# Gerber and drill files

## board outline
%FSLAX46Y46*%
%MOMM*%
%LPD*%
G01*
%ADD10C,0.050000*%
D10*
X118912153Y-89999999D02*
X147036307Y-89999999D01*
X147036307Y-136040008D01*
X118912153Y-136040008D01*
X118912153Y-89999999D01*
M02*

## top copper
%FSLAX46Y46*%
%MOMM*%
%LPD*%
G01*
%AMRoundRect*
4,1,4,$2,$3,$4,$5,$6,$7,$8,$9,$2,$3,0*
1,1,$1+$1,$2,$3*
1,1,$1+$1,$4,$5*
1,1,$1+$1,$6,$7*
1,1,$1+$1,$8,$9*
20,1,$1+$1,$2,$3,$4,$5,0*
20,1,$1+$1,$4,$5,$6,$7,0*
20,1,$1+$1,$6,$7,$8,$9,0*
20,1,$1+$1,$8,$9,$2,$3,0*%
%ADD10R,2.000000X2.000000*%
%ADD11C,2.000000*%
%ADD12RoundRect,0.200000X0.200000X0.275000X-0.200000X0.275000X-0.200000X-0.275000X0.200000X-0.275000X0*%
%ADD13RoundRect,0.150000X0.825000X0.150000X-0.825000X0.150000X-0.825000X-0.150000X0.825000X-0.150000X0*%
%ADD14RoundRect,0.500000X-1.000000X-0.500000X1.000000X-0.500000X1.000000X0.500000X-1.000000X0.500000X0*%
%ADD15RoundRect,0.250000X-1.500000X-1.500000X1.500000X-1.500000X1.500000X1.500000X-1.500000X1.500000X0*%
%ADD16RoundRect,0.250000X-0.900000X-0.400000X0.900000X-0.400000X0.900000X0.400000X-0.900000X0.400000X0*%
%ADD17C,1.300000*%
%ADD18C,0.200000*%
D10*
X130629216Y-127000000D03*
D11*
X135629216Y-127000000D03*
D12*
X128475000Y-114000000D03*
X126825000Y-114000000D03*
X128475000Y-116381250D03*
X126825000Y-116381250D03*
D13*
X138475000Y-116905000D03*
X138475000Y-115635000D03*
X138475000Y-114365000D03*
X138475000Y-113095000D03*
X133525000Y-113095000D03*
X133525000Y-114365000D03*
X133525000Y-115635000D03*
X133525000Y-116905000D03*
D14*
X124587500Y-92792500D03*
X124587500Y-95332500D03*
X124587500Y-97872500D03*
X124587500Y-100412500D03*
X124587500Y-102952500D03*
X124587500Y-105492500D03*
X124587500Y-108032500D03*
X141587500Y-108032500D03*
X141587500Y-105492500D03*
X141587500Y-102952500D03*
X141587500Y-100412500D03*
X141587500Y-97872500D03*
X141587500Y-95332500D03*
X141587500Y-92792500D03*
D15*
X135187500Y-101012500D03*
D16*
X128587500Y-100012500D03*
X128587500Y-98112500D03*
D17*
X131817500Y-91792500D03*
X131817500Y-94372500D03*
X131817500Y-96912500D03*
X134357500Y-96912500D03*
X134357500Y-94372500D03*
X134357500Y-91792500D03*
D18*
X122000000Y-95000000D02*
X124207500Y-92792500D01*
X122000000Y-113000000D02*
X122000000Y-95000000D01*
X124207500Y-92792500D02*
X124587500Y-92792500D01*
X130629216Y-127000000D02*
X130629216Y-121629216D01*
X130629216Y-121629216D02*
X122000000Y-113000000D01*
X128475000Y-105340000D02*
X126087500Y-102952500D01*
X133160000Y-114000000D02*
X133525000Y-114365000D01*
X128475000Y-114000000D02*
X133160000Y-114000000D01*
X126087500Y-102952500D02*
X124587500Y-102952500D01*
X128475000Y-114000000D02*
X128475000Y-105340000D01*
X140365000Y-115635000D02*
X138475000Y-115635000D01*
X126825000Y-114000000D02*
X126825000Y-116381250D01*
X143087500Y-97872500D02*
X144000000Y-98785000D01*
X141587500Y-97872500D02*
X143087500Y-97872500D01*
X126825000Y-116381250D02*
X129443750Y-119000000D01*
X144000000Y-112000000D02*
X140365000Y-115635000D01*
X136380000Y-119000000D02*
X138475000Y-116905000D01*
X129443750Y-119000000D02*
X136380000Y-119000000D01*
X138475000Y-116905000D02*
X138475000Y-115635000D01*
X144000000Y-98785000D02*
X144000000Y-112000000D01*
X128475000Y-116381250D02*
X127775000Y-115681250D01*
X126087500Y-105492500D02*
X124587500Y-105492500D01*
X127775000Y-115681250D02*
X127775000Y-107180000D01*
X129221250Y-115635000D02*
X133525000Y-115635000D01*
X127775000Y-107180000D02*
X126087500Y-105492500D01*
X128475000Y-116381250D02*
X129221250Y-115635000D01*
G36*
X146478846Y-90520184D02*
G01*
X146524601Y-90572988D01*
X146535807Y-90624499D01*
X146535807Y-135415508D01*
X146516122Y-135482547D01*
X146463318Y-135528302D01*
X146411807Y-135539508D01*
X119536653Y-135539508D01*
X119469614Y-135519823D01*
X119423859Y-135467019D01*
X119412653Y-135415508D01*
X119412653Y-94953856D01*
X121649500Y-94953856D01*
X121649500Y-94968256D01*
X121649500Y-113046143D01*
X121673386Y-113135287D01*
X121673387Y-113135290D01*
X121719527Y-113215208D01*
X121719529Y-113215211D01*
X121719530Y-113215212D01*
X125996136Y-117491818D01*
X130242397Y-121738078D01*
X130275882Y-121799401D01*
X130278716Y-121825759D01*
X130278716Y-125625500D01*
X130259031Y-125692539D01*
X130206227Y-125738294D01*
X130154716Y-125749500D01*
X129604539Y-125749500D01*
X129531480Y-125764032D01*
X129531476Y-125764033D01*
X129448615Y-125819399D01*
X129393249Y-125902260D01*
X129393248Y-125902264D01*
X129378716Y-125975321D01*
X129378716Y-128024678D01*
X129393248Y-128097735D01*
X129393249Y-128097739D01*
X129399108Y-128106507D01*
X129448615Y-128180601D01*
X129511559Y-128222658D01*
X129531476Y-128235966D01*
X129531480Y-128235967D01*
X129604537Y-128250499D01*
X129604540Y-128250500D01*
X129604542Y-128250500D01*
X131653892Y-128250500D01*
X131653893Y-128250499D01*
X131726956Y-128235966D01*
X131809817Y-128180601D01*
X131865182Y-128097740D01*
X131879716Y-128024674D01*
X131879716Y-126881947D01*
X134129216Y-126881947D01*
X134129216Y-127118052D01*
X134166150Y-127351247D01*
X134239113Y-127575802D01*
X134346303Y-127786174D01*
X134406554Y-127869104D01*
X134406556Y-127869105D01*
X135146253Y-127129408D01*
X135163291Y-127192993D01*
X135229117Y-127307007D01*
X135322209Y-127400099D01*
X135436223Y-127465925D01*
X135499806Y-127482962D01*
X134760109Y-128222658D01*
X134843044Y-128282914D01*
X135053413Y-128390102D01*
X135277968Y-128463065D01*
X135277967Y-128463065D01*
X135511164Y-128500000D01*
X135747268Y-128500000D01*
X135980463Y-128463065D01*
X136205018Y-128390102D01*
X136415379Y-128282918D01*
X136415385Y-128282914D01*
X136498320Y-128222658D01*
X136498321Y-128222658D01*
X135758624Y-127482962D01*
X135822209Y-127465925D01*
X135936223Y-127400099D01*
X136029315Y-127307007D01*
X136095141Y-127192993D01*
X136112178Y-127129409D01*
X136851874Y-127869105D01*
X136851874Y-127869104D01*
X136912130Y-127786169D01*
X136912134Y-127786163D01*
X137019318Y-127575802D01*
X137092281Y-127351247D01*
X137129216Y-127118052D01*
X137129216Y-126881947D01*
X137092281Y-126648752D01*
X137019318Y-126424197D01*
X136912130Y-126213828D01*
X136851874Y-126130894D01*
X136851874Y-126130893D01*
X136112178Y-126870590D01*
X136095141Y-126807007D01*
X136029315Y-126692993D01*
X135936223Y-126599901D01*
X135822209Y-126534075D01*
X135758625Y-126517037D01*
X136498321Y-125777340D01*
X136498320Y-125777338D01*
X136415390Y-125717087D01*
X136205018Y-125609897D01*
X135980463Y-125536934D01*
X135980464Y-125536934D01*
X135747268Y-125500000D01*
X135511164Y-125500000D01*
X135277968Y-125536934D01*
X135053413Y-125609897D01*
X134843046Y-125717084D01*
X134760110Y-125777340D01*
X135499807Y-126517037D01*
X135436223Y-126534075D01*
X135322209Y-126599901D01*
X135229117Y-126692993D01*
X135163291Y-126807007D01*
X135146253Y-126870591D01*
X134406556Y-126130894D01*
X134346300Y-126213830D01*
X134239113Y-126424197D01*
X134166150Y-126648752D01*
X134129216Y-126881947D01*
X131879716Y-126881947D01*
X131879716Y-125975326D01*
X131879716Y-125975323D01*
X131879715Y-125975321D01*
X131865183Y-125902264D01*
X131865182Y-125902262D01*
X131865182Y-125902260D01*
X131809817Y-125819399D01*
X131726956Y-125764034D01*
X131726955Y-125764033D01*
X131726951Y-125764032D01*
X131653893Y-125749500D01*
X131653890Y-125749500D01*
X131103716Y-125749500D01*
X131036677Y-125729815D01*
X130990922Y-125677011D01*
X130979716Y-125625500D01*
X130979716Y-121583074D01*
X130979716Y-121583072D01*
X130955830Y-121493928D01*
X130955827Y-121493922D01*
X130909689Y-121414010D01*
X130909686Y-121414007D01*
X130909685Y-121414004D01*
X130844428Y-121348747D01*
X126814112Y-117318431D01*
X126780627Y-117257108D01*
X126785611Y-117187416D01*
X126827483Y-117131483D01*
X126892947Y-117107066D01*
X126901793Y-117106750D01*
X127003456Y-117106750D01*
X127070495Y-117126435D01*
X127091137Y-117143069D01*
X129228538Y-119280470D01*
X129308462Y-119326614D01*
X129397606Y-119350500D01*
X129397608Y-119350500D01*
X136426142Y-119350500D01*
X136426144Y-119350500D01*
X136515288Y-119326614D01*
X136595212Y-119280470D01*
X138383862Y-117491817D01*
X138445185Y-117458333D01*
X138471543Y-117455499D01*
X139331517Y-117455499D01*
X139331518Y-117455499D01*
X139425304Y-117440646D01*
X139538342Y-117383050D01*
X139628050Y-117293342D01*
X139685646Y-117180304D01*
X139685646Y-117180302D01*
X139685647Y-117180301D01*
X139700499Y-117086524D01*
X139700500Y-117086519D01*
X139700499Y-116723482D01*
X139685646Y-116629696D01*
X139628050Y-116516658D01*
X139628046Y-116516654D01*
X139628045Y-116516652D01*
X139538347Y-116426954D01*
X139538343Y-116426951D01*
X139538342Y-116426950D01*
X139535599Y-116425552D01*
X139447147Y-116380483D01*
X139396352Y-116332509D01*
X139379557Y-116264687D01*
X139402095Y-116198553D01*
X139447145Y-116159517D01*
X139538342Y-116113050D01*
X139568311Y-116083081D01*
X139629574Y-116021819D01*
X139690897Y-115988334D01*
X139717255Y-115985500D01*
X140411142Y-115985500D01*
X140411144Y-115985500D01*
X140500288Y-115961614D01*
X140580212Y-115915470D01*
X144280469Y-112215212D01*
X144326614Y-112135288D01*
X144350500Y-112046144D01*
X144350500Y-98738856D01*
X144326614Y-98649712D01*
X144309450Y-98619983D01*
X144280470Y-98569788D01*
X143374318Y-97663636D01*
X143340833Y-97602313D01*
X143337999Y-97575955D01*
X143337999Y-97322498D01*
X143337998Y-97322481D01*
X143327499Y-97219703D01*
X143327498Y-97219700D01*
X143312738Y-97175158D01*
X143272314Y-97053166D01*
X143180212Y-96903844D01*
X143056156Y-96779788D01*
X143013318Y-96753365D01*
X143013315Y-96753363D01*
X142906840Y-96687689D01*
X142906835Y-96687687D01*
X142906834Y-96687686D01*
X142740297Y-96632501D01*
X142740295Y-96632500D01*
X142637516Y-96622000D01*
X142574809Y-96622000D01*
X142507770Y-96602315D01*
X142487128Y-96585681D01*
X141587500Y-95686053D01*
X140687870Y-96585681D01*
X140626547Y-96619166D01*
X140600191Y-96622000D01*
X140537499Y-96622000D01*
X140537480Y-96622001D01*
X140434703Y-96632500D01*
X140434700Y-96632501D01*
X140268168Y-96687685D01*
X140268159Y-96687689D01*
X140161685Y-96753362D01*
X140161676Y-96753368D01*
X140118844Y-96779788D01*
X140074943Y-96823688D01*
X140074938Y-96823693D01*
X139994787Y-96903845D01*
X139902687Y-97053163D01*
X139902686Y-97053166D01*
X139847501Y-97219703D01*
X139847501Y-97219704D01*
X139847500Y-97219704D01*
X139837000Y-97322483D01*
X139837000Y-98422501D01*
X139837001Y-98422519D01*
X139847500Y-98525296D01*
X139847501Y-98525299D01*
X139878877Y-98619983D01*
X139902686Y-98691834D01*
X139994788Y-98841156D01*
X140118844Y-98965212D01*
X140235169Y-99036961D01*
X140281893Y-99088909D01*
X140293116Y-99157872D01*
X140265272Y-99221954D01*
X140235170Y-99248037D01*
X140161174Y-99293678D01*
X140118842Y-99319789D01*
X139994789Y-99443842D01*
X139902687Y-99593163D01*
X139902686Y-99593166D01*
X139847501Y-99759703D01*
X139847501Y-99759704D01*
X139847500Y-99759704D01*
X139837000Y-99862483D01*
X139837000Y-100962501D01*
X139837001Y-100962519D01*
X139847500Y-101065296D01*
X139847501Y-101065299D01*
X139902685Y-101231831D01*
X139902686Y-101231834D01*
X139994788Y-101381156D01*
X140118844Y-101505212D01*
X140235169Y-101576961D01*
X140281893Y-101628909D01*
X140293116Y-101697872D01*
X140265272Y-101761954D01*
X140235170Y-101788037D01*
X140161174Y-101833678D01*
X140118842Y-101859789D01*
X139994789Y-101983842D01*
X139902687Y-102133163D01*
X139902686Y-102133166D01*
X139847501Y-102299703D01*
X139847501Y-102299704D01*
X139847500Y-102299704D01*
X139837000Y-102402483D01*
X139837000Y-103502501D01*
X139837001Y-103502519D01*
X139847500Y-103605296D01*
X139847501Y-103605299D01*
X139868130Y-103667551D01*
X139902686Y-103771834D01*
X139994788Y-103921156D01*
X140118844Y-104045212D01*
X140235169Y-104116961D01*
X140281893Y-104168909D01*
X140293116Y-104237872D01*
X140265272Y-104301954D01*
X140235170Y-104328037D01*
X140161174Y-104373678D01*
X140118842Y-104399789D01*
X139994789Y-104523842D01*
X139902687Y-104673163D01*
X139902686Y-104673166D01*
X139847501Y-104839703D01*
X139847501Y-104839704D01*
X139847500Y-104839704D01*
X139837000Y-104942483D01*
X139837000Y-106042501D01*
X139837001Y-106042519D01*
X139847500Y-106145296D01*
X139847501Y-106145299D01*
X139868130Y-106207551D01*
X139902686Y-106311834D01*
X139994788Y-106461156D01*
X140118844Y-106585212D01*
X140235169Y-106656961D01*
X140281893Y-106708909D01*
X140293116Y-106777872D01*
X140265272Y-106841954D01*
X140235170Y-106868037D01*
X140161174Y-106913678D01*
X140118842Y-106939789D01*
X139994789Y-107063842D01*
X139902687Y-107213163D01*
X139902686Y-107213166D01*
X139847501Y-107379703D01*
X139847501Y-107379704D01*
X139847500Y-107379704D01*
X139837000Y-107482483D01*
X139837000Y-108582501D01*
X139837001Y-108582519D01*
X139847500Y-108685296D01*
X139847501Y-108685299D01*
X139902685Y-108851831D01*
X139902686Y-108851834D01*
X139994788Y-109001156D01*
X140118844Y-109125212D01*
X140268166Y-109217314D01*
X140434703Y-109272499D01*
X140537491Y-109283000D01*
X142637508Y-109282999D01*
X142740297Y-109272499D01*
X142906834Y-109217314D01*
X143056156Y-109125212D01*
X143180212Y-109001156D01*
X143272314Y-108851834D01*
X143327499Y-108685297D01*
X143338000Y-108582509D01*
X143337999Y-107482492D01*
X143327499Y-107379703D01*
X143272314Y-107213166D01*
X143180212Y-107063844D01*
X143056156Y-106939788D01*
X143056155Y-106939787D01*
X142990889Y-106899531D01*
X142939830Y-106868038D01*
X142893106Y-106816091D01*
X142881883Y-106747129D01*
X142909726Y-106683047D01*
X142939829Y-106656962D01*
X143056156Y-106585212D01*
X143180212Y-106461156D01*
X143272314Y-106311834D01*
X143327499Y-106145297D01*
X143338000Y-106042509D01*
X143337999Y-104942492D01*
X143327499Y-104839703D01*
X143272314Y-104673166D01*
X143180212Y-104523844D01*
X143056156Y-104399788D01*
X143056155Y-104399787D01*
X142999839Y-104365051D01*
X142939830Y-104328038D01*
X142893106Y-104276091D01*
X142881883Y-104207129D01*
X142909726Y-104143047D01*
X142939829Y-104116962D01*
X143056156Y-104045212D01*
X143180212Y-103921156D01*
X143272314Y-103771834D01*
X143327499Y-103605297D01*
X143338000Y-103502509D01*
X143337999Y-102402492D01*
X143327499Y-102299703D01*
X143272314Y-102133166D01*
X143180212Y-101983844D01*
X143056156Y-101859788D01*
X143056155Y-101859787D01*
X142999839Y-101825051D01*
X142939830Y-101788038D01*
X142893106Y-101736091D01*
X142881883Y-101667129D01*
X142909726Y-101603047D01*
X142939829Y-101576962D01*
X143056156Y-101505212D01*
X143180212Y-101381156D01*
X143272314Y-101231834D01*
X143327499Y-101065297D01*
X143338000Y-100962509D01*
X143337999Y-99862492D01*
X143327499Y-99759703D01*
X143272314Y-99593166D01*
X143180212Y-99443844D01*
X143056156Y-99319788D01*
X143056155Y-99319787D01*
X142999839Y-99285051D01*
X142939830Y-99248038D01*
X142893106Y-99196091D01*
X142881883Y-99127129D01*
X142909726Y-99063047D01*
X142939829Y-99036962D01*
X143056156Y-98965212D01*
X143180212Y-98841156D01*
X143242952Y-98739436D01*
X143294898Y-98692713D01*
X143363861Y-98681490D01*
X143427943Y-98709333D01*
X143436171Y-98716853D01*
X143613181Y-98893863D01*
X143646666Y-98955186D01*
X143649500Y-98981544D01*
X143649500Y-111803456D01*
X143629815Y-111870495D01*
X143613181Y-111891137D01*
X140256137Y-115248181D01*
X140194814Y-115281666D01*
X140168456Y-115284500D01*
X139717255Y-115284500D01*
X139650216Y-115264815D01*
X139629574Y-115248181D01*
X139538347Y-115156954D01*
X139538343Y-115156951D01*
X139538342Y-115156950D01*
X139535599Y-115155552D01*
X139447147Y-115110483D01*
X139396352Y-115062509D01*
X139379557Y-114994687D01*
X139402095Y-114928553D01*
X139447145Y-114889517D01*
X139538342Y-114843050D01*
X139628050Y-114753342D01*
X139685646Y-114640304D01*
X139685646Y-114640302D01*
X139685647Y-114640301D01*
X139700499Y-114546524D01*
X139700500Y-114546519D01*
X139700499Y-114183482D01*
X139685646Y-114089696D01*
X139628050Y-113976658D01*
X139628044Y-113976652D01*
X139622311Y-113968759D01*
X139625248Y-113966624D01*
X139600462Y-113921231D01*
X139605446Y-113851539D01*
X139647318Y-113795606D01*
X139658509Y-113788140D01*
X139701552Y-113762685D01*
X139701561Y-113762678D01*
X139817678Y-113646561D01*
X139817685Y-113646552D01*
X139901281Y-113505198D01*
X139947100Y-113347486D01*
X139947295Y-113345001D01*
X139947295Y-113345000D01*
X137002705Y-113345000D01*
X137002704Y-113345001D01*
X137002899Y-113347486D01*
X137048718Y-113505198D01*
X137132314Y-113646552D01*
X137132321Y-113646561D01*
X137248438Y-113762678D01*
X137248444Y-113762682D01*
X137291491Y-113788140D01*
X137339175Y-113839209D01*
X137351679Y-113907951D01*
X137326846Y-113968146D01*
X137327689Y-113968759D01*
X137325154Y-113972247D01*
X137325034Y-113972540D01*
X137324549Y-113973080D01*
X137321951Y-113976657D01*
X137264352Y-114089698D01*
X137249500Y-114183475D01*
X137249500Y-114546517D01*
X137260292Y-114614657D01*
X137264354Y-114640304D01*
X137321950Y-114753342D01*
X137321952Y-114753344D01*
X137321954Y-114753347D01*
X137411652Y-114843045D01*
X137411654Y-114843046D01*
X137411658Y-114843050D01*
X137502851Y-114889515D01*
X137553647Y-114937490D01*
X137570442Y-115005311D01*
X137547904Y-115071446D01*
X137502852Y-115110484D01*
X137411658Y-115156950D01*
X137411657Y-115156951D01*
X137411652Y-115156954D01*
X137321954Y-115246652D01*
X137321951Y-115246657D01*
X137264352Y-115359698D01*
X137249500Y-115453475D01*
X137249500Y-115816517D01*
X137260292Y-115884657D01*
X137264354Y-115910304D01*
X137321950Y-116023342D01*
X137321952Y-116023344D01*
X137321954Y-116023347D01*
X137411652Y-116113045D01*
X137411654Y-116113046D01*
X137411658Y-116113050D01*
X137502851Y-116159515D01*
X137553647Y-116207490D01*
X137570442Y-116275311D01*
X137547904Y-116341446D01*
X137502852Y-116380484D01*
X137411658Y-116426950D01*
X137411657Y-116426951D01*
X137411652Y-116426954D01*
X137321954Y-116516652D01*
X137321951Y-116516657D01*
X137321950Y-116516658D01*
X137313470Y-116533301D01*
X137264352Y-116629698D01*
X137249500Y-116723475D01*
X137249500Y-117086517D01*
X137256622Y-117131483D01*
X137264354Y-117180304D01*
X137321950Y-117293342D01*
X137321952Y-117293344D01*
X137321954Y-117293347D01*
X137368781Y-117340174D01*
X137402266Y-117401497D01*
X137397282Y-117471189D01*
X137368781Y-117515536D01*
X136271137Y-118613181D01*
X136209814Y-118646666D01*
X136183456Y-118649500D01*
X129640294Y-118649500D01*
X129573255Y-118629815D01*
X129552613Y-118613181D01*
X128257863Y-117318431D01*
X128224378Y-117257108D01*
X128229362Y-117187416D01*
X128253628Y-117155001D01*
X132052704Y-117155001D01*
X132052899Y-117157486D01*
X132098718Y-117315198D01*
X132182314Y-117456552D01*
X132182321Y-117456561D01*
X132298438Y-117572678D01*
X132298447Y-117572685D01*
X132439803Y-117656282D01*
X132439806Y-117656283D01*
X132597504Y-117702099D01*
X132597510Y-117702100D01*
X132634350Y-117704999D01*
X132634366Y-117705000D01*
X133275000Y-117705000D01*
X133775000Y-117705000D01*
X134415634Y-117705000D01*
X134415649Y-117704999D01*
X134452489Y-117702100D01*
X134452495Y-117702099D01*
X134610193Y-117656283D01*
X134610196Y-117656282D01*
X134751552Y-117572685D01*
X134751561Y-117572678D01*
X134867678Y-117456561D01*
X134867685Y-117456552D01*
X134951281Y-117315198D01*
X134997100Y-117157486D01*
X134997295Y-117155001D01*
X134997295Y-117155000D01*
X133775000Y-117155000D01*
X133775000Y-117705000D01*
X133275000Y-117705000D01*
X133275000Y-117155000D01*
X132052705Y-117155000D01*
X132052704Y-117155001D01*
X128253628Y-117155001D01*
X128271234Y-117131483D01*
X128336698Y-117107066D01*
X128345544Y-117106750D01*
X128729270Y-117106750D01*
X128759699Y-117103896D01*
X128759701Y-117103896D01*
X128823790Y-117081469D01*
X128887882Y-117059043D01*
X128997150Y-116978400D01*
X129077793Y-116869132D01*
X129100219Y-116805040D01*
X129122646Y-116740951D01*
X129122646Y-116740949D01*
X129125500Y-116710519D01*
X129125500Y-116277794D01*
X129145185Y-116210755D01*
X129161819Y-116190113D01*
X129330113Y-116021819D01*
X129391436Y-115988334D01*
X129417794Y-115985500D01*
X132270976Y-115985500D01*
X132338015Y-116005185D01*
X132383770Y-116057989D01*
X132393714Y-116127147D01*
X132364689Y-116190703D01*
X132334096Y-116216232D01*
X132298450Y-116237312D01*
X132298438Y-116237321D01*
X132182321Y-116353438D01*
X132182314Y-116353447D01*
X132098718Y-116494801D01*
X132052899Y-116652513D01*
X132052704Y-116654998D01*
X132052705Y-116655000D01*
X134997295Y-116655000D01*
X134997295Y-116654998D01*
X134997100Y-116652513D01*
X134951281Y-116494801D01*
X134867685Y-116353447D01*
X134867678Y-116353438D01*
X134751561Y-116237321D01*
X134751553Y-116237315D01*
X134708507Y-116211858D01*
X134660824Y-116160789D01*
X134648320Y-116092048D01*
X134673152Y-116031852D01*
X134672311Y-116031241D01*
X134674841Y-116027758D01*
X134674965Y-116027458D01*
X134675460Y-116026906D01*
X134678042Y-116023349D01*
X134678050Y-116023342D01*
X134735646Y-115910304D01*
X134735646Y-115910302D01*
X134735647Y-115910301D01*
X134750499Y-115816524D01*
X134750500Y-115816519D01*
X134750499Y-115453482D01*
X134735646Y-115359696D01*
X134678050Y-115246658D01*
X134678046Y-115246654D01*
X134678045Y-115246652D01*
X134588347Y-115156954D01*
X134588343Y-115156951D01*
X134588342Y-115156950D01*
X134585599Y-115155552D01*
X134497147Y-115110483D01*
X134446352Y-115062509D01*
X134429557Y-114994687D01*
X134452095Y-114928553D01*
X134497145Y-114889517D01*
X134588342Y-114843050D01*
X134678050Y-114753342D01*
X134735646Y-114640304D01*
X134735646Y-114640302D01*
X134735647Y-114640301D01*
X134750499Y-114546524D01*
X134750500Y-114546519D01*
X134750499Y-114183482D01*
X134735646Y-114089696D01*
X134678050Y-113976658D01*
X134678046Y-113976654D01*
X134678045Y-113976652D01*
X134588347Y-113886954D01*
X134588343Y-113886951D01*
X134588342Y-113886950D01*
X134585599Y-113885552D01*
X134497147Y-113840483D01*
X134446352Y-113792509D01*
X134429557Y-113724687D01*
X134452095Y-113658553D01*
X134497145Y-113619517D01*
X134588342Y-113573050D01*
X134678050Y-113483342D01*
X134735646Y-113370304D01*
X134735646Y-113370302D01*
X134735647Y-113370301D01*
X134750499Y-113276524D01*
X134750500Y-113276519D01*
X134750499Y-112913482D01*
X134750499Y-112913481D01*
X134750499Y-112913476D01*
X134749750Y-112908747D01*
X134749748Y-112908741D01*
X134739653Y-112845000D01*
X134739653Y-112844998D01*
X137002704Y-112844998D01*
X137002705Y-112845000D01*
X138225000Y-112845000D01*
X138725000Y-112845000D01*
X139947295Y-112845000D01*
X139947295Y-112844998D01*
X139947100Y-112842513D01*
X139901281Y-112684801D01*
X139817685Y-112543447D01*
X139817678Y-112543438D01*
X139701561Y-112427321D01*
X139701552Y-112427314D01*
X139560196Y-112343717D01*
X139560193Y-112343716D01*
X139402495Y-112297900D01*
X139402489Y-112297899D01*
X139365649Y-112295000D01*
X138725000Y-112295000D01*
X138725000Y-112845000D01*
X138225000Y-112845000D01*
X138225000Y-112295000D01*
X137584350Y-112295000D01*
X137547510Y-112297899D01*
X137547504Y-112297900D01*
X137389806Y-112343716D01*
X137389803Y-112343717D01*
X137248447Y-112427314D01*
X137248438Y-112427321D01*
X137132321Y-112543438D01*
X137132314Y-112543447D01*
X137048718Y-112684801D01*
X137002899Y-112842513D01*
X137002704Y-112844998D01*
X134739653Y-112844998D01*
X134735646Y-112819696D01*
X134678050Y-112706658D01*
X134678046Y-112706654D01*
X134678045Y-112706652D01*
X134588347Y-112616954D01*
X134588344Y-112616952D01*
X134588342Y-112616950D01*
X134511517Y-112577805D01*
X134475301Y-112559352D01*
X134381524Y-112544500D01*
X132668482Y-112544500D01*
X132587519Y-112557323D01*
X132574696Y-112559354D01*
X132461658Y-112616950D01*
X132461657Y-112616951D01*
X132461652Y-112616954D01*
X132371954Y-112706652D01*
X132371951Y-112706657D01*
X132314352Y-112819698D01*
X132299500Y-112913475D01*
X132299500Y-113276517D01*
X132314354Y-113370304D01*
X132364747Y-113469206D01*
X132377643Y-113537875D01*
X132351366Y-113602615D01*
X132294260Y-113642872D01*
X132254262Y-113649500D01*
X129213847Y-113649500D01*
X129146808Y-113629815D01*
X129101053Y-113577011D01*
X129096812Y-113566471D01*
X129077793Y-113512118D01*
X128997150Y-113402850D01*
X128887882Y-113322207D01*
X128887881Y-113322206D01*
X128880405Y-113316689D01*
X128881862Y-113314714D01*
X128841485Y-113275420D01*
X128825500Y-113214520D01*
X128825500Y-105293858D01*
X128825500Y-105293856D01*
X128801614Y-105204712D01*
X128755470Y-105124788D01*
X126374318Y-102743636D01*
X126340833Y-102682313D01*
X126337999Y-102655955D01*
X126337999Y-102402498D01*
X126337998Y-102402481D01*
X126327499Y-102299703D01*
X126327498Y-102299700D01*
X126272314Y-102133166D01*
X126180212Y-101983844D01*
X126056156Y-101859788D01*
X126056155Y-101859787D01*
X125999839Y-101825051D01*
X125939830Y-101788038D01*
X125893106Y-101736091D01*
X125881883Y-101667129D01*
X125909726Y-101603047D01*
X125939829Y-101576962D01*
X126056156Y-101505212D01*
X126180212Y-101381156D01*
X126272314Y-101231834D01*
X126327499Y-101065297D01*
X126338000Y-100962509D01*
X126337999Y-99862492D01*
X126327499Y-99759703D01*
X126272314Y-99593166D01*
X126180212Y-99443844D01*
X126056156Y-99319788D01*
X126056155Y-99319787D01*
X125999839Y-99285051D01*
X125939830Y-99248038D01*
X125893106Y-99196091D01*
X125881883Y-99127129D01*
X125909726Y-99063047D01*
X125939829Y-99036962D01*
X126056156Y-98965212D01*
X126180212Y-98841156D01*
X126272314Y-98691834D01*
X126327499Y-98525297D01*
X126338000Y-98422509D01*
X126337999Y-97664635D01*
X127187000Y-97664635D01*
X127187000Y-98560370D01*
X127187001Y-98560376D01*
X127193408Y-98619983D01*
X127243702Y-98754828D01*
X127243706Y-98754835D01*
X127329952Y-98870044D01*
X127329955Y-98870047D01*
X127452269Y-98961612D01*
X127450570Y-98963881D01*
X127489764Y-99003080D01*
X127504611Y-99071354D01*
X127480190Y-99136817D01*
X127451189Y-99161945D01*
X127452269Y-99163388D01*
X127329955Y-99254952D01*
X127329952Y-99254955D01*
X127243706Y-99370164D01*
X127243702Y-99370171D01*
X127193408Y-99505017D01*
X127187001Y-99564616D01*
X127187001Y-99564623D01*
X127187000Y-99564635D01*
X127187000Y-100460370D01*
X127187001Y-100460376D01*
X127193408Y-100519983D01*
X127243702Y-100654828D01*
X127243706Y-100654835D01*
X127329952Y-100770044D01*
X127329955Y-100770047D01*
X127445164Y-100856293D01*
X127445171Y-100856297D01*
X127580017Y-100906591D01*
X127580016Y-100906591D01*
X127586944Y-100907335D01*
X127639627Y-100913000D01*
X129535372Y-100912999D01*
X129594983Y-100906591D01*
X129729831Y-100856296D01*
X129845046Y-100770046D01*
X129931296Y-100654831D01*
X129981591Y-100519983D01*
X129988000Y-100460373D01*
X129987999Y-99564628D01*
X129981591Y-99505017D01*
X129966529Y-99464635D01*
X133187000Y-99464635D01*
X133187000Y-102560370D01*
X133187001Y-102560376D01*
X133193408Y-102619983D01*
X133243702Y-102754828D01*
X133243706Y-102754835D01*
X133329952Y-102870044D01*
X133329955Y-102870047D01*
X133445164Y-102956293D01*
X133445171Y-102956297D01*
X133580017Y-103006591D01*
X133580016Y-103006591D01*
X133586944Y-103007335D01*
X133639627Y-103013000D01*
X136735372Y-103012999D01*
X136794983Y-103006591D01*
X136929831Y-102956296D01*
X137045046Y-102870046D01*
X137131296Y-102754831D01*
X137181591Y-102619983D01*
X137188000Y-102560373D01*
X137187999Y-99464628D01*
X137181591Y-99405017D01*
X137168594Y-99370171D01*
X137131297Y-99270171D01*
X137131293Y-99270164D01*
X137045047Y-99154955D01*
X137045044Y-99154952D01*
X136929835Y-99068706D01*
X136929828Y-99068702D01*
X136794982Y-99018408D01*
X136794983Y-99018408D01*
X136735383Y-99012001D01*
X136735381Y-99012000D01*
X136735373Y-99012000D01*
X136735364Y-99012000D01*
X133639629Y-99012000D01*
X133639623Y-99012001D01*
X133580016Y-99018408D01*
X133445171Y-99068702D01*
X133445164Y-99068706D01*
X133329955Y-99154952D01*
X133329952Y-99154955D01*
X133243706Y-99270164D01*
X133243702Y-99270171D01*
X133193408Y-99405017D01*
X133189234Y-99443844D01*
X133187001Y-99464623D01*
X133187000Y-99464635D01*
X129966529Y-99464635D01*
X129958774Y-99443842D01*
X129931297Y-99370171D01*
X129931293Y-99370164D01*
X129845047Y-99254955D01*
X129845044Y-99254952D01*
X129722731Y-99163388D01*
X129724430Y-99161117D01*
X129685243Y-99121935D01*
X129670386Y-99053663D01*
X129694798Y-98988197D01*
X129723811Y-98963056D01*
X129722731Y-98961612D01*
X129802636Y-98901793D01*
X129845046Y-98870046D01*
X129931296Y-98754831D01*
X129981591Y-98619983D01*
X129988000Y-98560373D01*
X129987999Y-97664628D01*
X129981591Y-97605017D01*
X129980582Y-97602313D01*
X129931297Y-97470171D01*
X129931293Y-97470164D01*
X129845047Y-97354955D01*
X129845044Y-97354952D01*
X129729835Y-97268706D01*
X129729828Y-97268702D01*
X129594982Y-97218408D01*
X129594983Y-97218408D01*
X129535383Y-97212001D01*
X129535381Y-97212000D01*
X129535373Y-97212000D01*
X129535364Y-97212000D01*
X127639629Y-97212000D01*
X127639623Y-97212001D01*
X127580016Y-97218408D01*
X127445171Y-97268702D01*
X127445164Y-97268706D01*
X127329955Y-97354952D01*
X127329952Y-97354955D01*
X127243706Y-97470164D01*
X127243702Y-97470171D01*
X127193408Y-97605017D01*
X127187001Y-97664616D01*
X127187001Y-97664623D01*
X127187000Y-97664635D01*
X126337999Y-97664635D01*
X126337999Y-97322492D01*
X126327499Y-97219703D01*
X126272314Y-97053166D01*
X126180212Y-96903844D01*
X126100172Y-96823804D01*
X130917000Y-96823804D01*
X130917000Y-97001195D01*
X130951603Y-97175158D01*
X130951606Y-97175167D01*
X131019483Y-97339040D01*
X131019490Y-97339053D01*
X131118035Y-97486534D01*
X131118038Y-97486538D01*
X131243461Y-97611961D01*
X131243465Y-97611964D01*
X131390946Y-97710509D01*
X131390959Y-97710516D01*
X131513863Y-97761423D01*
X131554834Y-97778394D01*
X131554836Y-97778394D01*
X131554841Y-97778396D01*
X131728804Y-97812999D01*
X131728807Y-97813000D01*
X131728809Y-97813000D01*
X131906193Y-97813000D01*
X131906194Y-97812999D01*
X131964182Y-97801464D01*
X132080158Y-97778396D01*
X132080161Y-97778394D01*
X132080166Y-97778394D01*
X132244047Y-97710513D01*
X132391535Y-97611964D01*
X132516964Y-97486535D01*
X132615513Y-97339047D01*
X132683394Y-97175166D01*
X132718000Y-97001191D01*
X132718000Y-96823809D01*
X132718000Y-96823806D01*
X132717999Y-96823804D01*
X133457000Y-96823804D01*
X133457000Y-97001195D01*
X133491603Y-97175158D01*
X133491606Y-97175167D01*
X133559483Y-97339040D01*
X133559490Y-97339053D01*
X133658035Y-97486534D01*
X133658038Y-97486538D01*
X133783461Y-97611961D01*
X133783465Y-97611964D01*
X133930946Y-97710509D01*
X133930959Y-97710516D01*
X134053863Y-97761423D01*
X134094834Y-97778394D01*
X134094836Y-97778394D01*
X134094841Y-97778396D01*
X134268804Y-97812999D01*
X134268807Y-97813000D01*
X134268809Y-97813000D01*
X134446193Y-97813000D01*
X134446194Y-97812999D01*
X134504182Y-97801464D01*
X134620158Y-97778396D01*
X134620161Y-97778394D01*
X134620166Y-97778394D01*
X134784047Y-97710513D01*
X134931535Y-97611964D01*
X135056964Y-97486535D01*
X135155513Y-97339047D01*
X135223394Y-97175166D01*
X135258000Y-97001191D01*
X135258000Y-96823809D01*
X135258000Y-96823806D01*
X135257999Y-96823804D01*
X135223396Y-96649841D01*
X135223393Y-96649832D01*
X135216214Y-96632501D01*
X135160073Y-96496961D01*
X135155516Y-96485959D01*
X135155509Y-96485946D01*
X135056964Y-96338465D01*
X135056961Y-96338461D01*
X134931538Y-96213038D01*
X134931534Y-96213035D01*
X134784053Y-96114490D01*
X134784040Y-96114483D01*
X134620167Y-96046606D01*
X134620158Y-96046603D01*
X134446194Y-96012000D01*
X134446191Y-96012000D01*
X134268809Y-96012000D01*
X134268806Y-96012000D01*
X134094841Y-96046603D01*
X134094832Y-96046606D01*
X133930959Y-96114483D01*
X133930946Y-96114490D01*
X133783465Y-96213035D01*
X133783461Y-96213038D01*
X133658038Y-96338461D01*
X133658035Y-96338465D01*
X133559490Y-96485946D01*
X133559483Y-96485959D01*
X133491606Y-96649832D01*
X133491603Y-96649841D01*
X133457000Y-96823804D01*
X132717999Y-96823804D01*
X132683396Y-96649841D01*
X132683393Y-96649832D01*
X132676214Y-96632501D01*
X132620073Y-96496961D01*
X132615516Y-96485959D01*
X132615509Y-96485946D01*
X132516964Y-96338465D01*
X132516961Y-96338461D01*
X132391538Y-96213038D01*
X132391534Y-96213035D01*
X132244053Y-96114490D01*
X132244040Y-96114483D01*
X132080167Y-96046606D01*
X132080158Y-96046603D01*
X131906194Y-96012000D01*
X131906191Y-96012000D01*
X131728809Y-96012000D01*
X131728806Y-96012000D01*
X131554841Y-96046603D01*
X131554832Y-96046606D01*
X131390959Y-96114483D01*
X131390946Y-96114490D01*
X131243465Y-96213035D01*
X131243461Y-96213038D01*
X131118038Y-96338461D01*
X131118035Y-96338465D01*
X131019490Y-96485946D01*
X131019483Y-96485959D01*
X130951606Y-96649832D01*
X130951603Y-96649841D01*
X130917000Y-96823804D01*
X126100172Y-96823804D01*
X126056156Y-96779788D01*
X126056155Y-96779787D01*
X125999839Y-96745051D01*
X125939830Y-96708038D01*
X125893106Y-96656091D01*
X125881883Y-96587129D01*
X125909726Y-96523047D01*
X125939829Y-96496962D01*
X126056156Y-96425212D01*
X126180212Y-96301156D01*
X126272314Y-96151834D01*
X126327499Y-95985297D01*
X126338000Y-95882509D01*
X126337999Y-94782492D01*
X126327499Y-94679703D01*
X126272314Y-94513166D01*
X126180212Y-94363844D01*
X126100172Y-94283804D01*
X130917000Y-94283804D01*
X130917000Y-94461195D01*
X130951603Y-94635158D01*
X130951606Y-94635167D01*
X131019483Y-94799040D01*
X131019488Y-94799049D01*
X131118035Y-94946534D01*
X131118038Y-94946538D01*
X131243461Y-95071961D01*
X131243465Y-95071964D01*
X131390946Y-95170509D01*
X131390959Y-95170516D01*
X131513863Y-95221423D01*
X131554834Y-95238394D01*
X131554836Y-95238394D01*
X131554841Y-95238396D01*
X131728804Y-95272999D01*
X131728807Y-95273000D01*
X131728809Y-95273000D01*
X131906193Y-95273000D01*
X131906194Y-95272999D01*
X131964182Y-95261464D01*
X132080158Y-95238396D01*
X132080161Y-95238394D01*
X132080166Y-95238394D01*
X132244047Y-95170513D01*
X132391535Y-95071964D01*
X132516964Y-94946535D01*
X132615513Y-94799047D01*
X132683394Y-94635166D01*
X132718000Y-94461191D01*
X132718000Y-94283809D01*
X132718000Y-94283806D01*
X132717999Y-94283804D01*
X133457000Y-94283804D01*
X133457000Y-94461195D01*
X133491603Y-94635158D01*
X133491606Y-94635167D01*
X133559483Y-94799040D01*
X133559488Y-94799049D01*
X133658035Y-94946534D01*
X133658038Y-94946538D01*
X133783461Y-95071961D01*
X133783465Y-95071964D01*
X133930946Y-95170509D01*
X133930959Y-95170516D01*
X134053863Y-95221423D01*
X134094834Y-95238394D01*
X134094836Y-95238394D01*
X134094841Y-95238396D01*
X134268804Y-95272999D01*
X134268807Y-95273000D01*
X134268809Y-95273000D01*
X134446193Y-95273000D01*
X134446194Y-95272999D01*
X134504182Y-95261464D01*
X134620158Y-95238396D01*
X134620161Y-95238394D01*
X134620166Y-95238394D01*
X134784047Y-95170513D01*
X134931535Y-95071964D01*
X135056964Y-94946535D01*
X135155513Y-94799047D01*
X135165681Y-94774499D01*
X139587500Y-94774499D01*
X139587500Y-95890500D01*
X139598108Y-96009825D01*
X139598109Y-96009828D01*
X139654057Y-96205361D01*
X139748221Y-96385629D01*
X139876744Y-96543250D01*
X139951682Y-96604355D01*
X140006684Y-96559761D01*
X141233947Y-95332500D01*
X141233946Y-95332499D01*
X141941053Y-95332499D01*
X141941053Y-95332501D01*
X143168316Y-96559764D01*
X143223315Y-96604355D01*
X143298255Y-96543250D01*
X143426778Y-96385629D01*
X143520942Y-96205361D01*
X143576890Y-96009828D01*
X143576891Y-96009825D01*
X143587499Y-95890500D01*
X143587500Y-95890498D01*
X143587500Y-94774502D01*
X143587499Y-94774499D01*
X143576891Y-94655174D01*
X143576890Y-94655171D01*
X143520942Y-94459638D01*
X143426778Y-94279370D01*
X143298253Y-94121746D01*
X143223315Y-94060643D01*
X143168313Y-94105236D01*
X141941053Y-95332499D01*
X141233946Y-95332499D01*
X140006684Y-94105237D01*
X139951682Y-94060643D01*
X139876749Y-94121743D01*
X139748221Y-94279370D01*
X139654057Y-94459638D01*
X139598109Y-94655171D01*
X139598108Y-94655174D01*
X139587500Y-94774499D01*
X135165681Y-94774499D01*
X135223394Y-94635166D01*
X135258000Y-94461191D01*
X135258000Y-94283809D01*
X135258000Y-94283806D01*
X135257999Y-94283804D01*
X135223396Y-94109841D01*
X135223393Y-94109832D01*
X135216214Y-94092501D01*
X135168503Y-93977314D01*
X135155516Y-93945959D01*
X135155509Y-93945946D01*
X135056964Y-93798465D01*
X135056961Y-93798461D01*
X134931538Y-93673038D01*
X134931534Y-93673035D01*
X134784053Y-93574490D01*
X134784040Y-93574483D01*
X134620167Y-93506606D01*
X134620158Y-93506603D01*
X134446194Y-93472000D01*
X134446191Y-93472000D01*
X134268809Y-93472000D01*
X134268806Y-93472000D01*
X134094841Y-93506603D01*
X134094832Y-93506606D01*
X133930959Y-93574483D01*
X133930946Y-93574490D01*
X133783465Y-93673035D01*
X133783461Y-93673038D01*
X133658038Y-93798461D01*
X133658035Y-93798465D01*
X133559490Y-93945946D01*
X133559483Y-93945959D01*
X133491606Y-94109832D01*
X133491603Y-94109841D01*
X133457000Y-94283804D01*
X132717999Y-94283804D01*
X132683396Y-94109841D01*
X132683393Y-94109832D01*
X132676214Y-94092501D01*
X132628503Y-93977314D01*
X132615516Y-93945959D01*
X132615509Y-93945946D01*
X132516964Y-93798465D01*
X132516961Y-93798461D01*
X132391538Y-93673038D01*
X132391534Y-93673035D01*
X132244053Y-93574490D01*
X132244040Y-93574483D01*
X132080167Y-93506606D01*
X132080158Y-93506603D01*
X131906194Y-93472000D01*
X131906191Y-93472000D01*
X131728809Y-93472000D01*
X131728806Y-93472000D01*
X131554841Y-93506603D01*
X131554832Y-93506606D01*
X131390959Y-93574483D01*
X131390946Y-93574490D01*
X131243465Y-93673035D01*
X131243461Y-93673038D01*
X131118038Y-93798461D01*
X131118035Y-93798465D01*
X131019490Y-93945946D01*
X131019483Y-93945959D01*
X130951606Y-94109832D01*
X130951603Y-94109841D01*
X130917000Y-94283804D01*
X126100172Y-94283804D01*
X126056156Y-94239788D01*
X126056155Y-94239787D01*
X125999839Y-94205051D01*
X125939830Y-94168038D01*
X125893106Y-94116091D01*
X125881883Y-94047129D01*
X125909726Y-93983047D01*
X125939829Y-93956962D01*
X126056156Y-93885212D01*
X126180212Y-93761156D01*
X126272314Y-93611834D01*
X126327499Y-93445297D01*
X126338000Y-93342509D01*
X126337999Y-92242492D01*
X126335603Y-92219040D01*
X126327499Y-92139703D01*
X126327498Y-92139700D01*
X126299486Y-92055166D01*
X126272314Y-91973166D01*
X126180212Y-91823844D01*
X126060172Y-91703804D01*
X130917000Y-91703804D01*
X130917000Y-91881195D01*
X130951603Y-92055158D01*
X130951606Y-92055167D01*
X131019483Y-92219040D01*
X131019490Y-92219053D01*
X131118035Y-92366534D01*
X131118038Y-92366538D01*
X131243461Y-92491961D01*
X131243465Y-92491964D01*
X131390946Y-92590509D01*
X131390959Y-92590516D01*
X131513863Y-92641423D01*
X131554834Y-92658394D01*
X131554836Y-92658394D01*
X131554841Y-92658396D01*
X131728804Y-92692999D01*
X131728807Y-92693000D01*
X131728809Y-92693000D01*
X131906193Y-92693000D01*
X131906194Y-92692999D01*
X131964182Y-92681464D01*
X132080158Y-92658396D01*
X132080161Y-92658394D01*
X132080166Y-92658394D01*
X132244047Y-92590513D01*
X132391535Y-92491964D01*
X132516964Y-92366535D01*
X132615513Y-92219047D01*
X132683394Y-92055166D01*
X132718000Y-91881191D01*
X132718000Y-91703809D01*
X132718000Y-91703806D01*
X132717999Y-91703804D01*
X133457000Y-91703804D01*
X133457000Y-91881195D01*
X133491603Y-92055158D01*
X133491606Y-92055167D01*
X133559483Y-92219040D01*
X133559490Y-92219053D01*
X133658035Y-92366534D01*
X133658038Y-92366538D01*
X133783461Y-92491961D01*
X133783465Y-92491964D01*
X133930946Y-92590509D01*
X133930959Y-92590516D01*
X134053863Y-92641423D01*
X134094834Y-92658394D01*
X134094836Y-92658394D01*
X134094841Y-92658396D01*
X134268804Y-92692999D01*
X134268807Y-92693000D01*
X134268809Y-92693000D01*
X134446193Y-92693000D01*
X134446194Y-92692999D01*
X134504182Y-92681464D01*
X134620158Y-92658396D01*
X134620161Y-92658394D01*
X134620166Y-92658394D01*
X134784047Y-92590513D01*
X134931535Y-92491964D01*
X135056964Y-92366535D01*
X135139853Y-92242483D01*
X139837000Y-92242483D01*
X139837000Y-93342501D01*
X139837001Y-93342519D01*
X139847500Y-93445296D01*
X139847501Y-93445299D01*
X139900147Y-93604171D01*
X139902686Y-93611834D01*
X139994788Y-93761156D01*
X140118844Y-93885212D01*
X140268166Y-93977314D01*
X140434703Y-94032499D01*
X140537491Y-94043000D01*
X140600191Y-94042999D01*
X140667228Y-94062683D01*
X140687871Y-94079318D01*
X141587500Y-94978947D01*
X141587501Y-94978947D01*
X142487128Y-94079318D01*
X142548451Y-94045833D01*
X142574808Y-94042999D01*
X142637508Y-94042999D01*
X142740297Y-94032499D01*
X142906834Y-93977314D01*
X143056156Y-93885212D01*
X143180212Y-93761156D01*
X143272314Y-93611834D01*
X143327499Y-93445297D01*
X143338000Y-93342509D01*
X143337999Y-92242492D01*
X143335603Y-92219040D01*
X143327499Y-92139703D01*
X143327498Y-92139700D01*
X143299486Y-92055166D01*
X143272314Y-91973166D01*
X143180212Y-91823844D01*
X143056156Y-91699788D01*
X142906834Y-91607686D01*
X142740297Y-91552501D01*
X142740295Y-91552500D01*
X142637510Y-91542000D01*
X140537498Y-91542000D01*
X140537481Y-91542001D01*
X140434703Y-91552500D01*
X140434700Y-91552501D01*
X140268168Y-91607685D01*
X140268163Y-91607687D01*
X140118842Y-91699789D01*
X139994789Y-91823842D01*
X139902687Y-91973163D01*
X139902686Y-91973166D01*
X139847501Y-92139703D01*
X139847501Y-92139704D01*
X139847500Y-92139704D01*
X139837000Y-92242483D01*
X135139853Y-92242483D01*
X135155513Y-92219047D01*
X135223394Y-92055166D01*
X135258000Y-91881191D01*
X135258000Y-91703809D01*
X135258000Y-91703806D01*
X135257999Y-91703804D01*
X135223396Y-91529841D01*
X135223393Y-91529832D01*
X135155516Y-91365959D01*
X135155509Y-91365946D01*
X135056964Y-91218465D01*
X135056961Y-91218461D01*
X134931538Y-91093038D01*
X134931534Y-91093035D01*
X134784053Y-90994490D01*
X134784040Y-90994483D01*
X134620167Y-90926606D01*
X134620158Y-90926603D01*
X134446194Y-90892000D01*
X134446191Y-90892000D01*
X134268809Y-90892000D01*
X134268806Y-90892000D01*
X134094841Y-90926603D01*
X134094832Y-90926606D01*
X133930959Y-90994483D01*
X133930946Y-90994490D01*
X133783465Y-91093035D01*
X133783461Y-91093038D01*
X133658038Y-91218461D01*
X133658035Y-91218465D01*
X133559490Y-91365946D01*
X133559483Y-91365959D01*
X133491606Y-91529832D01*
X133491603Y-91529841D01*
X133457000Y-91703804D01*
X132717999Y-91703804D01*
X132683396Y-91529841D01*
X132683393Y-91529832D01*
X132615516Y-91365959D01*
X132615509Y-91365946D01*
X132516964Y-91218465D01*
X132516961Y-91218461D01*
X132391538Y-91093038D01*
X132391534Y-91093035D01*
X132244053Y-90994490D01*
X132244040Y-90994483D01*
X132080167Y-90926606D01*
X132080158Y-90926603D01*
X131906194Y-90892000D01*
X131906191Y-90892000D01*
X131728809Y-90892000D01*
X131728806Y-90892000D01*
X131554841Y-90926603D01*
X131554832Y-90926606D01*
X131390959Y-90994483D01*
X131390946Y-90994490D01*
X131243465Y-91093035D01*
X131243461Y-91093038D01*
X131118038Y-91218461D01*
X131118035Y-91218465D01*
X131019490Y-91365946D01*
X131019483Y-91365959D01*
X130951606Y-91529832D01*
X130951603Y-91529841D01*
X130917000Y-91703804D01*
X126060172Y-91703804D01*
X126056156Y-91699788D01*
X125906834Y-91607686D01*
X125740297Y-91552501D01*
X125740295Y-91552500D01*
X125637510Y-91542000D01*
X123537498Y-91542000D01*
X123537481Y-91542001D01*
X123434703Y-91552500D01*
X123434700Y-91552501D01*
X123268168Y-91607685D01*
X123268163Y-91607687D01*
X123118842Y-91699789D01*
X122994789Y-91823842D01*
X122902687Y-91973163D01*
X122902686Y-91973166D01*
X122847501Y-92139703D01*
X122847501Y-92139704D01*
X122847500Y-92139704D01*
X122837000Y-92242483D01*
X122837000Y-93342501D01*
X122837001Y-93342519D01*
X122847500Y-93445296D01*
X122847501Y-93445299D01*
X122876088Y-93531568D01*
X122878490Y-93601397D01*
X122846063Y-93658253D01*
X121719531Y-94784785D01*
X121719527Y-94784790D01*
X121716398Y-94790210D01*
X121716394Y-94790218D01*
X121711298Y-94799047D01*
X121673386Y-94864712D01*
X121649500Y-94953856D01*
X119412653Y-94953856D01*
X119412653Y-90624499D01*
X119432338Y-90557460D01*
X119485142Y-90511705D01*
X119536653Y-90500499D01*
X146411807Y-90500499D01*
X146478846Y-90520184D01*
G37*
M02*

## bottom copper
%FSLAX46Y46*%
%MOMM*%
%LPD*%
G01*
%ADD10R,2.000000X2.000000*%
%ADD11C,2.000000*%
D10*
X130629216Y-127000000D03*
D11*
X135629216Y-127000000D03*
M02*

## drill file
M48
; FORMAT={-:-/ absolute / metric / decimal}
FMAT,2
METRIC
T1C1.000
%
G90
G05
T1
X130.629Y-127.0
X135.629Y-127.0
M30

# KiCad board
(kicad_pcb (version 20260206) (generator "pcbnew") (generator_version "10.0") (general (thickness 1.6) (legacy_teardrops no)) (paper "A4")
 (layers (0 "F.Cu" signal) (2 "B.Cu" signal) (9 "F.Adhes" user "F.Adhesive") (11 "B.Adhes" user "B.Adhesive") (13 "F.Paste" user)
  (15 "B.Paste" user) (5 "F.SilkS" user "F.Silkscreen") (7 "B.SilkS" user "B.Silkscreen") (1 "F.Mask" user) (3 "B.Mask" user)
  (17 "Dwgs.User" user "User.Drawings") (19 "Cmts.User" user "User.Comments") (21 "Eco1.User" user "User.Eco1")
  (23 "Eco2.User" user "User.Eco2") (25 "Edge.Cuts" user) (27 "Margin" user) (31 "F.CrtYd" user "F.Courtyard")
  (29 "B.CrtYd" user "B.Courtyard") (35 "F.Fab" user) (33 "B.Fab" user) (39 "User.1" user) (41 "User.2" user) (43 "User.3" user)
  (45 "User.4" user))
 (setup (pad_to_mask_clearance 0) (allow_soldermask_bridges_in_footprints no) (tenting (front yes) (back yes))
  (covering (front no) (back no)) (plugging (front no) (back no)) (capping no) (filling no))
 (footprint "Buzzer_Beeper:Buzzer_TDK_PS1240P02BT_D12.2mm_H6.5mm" (layer "F.Cu") (at 130.629216 127)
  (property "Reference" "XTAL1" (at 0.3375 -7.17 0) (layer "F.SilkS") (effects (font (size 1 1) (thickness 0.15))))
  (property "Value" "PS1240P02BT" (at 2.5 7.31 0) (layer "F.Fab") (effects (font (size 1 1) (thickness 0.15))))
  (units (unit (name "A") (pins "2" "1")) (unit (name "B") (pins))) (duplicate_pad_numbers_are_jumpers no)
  (pad "1" thru_hole rect (at 0 0) (size 2 2) (drill 1) (layers "*.Cu" "*.Mask") (remove_unused_layers no) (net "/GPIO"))
  (pad "2" thru_hole circle (at 5 0) (size 2 2) (drill 1) (layers "*.Cu" "*.Mask") (remove_unused_layers no) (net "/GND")))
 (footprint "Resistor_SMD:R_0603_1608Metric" (layer "F.Cu") (at 127.65 114 180)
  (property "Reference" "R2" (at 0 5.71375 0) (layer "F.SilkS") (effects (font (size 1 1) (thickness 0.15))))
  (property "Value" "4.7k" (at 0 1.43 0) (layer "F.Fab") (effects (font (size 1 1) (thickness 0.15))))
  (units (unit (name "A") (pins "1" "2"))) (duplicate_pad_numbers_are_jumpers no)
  (pad "1" smd roundrect (at -0.825 0 180) (size 0.8 0.95) (layers "F.Cu" "F.Mask" "F.Paste") (roundrect_rratio 0.25) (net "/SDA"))
  (pad "2" smd roundrect (at 0.825 0 180) (size 0.8 0.95) (layers "F.Cu" "F.Mask" "F.Paste") (roundrect_rratio 0.25) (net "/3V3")))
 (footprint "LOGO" (layer "F.Cu") (at 142 120 90)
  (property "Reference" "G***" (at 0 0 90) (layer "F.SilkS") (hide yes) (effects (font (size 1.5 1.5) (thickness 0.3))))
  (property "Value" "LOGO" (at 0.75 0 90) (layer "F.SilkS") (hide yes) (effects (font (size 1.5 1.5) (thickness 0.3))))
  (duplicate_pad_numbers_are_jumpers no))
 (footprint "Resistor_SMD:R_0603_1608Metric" (layer "F.Cu") (at 127.65 116.38125 180)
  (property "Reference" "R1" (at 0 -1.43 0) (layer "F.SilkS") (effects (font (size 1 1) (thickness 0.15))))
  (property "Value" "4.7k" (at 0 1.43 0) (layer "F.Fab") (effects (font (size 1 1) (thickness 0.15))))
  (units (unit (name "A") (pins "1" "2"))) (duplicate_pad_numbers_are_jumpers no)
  (pad "1" smd roundrect (at -0.825 0 180) (size 0.8 0.95) (layers "F.Cu" "F.Mask" "F.Paste") (roundrect_rratio 0.25) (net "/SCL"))
  (pad "2" smd roundrect (at 0.825 0 180) (size 0.8 0.95) (layers "F.Cu" "F.Mask" "F.Paste") (roundrect_rratio 0.25) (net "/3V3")))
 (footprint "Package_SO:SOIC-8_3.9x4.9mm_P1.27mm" (layer "F.Cu") (at 136 115 180)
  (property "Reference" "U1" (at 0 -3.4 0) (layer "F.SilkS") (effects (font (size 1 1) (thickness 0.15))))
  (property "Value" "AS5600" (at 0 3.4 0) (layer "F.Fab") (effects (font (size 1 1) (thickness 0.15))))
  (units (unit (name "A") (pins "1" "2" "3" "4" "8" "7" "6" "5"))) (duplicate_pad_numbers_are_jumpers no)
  (pad "1" smd roundrect (at -2.475 -1.905 180) (size 1.95 0.6) (layers "F.Cu" "F.Mask" "F.Paste") (roundrect_rratio 0.25) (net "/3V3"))
  (pad "2" smd roundrect (at -2.475 -0.635 180) (size 1.95 0.6) (layers "F.Cu" "F.Mask" "F.Paste") (roundrect_rratio 0.25) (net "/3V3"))
  (pad "3" smd roundrect (at -2.475 0.635 180) (size 1.95 0.6) (layers "F.Cu" "F.Mask" "F.Paste") (roundrect_rratio 0.25)
   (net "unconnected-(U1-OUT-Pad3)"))
  (pad "4" smd roundrect (at -2.475 1.905 180) (size 1.95 0.6) (layers "F.Cu" "F.Mask" "F.Paste") (roundrect_rratio 0.25) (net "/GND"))
  (pad "5" smd roundrect (at 2.475 1.905 180) (size 1.95 0.6) (layers "F.Cu" "F.Mask" "F.Paste") (roundrect_rratio 0.25)
   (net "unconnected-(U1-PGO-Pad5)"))
  (pad "6" smd roundrect (at 2.475 0.635 180) (size 1.95 0.6) (layers "F.Cu" "F.Mask" "F.Paste") (roundrect_rratio 0.25) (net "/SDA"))
  (pad "7" smd roundrect (at 2.475 -0.635 180) (size 1.95 0.6) (layers "F.Cu" "F.Mask" "F.Paste") (roundrect_rratio 0.25) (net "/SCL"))
  (pad "8" smd roundrect (at 2.475 -1.905 180) (size 1.95 0.6) (layers "F.Cu" "F.Mask" "F.Paste") (roundrect_rratio 0.25) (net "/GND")))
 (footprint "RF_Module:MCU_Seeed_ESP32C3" (layer "F.Cu") (at 133.0875 100.4125)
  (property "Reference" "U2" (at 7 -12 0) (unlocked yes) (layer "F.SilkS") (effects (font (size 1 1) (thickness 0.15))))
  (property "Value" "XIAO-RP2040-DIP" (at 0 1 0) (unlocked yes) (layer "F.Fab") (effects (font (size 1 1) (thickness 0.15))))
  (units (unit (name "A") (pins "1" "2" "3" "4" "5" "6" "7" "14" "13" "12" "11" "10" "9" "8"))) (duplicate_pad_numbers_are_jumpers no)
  (pad "" smd roundrect (at 1.1 -0.4) (size 1.5 1.5) (layers "F.Paste") (roundrect_rratio 0.1666666667))
  (pad "" smd roundrect (at 1.1 1.6) (size 1.5 1.5) (layers "F.Paste") (roundrect_rratio 0.1666666667))
  (pad "" smd roundrect (at 3.1 -0.4) (size 1.5 1.5) (layers "F.Paste") (roundrect_rratio 0.1666666667))
  (pad "" smd roundrect (at 3.1 1.6) (size 1.5 1.5) (layers "F.Paste") (roundrect_rratio 0.1666666667))
  (pad "1" smd roundrect (at -8.5 -7.62) (size 3 2) (layers "F.Cu" "F.Mask" "F.Paste") (roundrect_rratio 0.25) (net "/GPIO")
   (thermal_bridge_angle 45))
  (pad "2" smd roundrect (at -8.5 -5.08) (size 3 2) (layers "F.Cu" "F.Mask" "F.Paste") (roundrect_rratio 0.25)
   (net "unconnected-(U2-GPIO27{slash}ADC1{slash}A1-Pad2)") (thermal_bridge_angle 45))
  (pad "3" smd roundrect (at -8.5 -2.54) (size 3 2) (layers "F.Cu" "F.Mask" "F.Paste") (roundrect_rratio 0.25)
   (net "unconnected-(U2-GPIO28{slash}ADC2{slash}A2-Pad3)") (thermal_bridge_angle 45))
  (pad "4" smd roundrect (at -8.5 0) (size 3 2) (layers "F.Cu" "F.Mask" "F.Paste") (roundrect_rratio 0.25)
   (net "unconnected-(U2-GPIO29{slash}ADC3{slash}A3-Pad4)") (thermal_bridge_angle 45))
  (pad "5" smd roundrect (at -8.5 2.54) (size 3 2) (layers "F.Cu" "F.Mask" "F.Paste") (roundrect_rratio 0.25) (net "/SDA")
   (thermal_bridge_angle 45))
  (pad "6" smd roundrect (at -8.5 5.08) (size 3 2) (layers "F.Cu" "F.Mask" "F.Paste") (roundrect_rratio 0.25) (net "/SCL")
   (thermal_bridge_angle 45))
  (pad "7" smd roundrect (at -8.5 7.62) (size 3 2) (layers "F.Cu" "F.Mask" "F.Paste") (roundrect_rratio 0.25)
   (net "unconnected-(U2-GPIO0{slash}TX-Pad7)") (thermal_bridge_angle 45))
  (pad "8" smd roundrect (at 8.5 7.62) (size 3 2) (layers "F.Cu" "F.Mask" "F.Paste") (roundrect_rratio 0.25)
   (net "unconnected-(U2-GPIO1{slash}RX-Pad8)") (thermal_bridge_angle 45))
  (pad "9" smd roundrect (at 8.5 5.08) (size 3 2) (layers "F.Cu" "F.Mask" "F.Paste") (roundrect_rratio 0.25)
   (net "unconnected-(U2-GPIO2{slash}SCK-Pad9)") (thermal_bridge_angle 45))
  (pad "10" smd roundrect (at 8.5 2.54) (size 3 2) (layers "F.Cu" "F.Mask" "F.Paste") (roundrect_rratio 0.25)
   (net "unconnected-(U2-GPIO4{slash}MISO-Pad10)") (thermal_bridge_angle 45))
  (pad "11" smd roundrect (at 8.5 0) (size 3 2) (layers "F.Cu" "F.Mask" "F.Paste") (roundrect_rratio 0.25)
   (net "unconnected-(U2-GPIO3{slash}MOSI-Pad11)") (thermal_bridge_angle 45))
  (pad "12" smd roundrect (at 8.5 -2.54) (size 3 2) (layers "F.Cu" "F.Mask" "F.Paste") (roundrect_rratio 0.25) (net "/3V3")
   (thermal_bridge_angle 45))
  (pad "13" smd roundrect (at 8.5 -5.08) (size 3 2) (layers "F.Cu" "F.Mask" "F.Paste") (roundrect_rratio 0.25) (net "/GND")
   (thermal_bridge_angle 45))
  (pad "14" smd roundrect (at 8.5 -7.62) (size 3 2) (layers "F.Cu" "F.Mask" "F.Paste") (roundrect_rratio 0.25)
   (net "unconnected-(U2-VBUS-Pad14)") (thermal_bridge_angle 45))
  (pad "15" smd roundrect (at 2.1 0.6) (size 3.5 3.5) (layers "F.Cu" "F.Mask") (roundrect_rratio 0.07142857143))
  (pad "16" smd roundrect (at -4.5 -0.4) (size 2.3 1.3) (layers "F.Cu" "F.Mask" "F.Paste") (roundrect_rratio 0.1923076923))
  (pad "17" smd roundrect (at -4.5 -2.3) (size 2.3 1.3) (layers "F.Cu" "F.Mask" "F.Paste") (roundrect_rratio 0.1923076923))
  (pad "18" smd circle (at -1.27 -8.62) (size 1.3 1.3) (layers "F.Cu" "F.Mask" "F.Paste"))
  (pad "19" smd circle (at -1.27 -6.04) (size 1.3 1.3) (layers "F.Cu" "F.Mask" "F.Paste"))
  (pad "20" smd circle (at -1.27 -3.5) (size 1.3 1.3) (layers "F.Cu" "F.Mask" "F.Paste"))
  (pad "21" smd circle (at 1.27 -3.5) (size 1.3 1.3) (layers "F.Cu" "F.Mask" "F.Paste"))
  (pad "22" smd circle (at 1.27 -6.04) (size 1.3 1.3) (layers "F.Cu" "F.Mask" "F.Paste"))
  (pad "23" smd circle (at 1.27 -8.62) (size 1.3 1.3) (layers "F.Cu" "F.Mask" "F.Paste")))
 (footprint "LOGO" (layer "F.Cu") (at 143 129 90)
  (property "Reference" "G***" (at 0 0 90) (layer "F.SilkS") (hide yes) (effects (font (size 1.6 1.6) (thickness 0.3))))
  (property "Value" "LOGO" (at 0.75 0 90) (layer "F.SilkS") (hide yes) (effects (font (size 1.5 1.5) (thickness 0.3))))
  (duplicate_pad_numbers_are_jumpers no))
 (gr_rect (start 118.912153 89.999999) (end 147.036307 136.040008) (stroke (width 0.05) (type default)) (fill no) (layer "Edge.Cuts"))
 (segment (start 122 95) (end 124.2075 92.7925) (width 0.2) (layer "F.Cu") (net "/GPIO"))
 (segment (start 122 113) (end 122 95) (width 0.2) (layer "F.Cu") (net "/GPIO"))
 (segment (start 124.2075 92.7925) (end 124.5875 92.7925) (width 0.2) (layer "F.Cu") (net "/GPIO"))
 (segment (start 130.629216 127) (end 130.629216 121.629216) (width 0.2) (layer "F.Cu") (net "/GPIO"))
 (segment (start 130.629216 121.629216) (end 122 113) (width 0.2) (layer "F.Cu") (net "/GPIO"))
 (segment (start 128.475 105.34) (end 126.0875 102.9525) (width 0.2) (layer "F.Cu") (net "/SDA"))
 (segment (start 133.16 114) (end 133.525 114.365) (width 0.2) (layer "F.Cu") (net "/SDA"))
 (segment (start 128.475 114) (end 133.16 114) (width 0.2) (layer "F.Cu") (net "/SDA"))
 (segment (start 126.0875 102.9525) (end 124.5875 102.9525) (width 0.2) (layer "F.Cu") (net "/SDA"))
 (segment (start 128.475 114) (end 128.475 105.34) (width 0.2) (layer "F.Cu") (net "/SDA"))
 (segment (start 140.365 115.635) (end 138.475 115.635) (width 0.2) (layer "F.Cu") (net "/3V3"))
 (segment (start 126.825 114) (end 126.825 116.38125) (width 0.2) (layer "F.Cu") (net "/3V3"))
 (segment (start 143.0875 97.8725) (end 144 98.785) (width 0.2) (layer "F.Cu") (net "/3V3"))
 (segment (start 141.5875 97.8725) (end 143.0875 97.8725) (width 0.2) (layer "F.Cu") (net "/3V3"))
 (segment (start 126.825 116.38125) (end 129.44375 119) (width 0.2) (layer "F.Cu") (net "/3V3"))
 (segment (start 144 112) (end 140.365 115.635) (width 0.2) (layer "F.Cu") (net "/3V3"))
 (segment (start 136.38 119) (end 138.475 116.905) (width 0.2) (layer "F.Cu") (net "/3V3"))
 (segment (start 129.44375 119) (end 136.38 119) (width 0.2) (layer "F.Cu") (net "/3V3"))
 (segment (start 138.475 116.905) (end 138.475 115.635) (width 0.2) (layer "F.Cu") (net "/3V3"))
 (segment (start 144 98.785) (end 144 112) (width 0.2) (layer "F.Cu") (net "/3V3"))
 (segment (start 128.475 116.38125) (end 127.775 115.68125) (width 0.2) (layer "F.Cu") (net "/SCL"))
 (segment (start 126.0875 105.4925) (end 124.5875 105.4925) (width 0.2) (layer "F.Cu") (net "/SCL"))
 (segment (start 127.775 115.68125) (end 127.775 107.18) (width 0.2) (layer "F.Cu") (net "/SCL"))
 (segment (start 129.22125 115.635) (end 133.525 115.635) (width 0.2) (layer "F.Cu") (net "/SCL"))
 (segment (start 127.775 107.18) (end 126.0875 105.4925) (width 0.2) (layer "F.Cu") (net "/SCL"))
 (segment (start 128.475 116.38125) (end 129.22125 115.635) (width 0.2) (layer "F.Cu") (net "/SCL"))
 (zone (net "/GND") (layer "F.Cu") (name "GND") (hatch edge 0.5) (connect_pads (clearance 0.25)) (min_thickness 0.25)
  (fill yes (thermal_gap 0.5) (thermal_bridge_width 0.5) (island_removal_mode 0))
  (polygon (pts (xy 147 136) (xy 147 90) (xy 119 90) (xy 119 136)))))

